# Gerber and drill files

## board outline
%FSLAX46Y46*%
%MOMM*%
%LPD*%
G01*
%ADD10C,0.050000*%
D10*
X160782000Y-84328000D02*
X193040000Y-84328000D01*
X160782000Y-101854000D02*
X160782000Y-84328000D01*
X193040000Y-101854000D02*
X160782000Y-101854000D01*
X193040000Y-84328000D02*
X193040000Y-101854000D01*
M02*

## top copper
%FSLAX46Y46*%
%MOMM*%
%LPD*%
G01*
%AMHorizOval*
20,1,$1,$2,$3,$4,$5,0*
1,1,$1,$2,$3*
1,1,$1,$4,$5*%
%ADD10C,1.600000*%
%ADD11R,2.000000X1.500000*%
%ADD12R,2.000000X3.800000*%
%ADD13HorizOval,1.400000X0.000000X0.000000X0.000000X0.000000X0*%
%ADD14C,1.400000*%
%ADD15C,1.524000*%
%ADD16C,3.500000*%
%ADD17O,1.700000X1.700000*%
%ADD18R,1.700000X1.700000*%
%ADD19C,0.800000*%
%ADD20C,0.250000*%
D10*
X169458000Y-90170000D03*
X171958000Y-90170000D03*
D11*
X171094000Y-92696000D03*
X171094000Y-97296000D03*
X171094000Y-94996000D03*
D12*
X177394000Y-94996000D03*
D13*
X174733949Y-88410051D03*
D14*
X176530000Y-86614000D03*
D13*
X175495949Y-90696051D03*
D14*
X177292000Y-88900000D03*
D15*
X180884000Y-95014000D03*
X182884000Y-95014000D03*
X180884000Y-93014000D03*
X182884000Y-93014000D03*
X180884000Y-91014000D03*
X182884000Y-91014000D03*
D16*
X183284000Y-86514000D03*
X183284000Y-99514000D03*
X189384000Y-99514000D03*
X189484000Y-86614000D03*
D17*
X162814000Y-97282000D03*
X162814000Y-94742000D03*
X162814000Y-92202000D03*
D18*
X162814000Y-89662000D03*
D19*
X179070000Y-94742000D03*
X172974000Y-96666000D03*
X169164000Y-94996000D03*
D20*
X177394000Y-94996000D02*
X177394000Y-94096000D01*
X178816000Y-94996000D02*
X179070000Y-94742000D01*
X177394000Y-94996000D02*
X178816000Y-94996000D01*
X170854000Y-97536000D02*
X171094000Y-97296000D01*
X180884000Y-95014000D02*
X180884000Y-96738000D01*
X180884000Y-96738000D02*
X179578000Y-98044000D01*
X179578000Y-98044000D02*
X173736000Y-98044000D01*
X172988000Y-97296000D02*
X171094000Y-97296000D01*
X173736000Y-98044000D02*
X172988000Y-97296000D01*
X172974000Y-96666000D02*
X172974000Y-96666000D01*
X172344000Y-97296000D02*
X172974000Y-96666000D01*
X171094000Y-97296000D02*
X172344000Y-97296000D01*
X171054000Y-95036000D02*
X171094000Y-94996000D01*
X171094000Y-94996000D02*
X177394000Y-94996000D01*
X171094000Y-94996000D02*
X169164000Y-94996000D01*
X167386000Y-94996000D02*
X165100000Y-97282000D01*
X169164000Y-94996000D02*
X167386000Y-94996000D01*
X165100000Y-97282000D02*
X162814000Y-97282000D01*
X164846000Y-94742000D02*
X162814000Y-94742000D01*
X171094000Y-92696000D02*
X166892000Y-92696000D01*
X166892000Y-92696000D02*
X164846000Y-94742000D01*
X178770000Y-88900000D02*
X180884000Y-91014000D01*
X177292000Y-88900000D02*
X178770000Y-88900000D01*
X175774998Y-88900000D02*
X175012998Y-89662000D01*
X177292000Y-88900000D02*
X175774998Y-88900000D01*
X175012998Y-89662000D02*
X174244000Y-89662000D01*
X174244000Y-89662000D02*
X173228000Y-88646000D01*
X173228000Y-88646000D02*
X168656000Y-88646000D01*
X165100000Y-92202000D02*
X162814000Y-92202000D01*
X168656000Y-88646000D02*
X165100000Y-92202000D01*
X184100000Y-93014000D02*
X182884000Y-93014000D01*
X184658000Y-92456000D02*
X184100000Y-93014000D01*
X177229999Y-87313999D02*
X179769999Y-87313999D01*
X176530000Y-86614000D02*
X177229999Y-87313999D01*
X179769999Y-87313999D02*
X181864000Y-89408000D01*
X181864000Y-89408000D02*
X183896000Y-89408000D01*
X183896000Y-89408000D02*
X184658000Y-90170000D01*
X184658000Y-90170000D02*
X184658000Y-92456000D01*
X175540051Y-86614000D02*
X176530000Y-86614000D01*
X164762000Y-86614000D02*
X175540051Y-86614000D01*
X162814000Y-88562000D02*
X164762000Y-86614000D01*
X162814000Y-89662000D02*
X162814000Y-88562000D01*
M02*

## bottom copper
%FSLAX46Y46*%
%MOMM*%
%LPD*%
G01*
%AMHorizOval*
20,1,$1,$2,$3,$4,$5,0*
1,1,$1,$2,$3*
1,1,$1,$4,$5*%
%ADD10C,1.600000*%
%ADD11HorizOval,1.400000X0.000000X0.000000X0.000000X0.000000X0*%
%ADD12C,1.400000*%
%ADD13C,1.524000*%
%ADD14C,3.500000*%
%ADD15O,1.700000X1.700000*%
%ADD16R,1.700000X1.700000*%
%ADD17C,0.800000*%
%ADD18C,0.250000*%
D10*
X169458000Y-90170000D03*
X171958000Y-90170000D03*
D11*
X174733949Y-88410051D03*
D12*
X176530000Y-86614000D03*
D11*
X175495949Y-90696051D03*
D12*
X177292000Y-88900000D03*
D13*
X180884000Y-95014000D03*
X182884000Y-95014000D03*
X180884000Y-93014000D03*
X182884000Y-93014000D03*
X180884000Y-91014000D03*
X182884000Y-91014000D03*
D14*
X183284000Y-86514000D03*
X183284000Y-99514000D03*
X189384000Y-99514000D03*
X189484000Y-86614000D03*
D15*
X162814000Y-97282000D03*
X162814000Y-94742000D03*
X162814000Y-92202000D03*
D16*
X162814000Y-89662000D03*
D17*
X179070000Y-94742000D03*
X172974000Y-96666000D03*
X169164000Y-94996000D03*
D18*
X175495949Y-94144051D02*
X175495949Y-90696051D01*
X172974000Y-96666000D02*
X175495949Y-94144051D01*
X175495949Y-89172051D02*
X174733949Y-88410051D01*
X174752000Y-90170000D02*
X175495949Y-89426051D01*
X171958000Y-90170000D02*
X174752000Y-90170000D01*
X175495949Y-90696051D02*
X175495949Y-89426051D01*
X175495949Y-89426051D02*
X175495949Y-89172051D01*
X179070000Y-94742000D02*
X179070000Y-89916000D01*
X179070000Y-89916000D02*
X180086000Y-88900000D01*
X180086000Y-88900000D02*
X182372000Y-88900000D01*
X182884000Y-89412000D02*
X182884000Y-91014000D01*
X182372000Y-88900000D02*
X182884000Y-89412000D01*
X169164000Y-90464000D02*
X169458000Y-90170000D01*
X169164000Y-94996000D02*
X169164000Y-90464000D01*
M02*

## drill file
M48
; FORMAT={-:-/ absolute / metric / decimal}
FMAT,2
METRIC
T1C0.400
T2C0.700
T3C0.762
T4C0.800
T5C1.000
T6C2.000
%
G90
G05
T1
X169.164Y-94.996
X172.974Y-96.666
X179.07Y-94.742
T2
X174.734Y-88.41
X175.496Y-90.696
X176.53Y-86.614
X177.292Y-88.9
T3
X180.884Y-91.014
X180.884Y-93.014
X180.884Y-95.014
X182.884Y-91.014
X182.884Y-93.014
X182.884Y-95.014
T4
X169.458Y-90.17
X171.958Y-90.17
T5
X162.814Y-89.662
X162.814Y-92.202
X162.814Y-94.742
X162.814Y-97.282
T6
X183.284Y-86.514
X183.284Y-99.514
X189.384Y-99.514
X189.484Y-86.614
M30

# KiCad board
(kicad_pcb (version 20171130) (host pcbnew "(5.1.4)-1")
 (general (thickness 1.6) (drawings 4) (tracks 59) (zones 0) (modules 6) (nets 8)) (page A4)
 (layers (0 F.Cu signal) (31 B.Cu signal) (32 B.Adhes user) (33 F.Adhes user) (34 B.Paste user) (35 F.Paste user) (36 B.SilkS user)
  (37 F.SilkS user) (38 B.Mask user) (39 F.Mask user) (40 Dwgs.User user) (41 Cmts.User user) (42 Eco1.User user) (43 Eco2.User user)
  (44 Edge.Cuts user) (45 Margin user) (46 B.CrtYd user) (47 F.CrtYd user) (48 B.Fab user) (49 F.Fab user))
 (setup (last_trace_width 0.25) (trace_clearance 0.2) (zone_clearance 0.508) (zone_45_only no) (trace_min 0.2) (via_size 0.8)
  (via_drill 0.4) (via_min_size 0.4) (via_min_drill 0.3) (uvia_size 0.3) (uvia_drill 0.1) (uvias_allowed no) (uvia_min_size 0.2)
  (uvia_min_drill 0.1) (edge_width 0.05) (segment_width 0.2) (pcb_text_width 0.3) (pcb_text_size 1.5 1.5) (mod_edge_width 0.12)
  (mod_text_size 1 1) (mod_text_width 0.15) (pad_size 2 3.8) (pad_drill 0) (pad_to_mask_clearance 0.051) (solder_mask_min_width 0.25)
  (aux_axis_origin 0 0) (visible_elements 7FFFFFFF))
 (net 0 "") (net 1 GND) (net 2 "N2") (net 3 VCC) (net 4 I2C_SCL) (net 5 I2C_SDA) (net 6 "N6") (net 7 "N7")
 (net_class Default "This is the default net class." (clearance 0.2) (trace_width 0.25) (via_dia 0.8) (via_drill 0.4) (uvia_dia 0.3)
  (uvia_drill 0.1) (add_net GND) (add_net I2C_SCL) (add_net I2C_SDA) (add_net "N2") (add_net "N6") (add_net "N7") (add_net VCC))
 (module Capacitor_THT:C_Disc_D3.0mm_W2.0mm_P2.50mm (layer F.Cu) (at 171.958 90.17 180)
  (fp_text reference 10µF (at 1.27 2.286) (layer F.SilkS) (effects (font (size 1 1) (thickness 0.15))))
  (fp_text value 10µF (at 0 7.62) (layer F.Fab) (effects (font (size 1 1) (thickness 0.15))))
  (pad 2 thru_hole circle (at 2.5 0 180) (size 1.6 1.6) (drill 0.8) (layers *.Cu *.Mask) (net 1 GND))
  (pad 1 thru_hole circle (at 0 0 180) (size 1.6 1.6) (drill 0.8) (layers *.Cu *.Mask) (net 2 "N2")))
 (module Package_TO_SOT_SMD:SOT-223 (layer F.Cu) (at 174.244 94.996)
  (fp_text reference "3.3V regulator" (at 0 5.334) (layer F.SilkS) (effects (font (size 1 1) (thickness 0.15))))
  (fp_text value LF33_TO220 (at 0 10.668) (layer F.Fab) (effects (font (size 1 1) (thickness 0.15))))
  (pad 1 smd rect (at -3.15 -2.3) (size 2 1.5) (layers F.Cu F.Paste F.Mask) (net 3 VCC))
  (pad 3 smd rect (at -3.15 2.3) (size 2 1.5) (layers F.Cu F.Paste F.Mask) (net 2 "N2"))
  (pad 2 smd rect (at -3.15 0) (size 2 1.5) (layers F.Cu F.Paste F.Mask) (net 1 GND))
  (pad 4 smd rect (at 3.15 0) (size 2 3.8) (layers F.Cu F.Paste F.Mask) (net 1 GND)))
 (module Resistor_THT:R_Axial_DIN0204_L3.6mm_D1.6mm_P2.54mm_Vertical (layer F.Cu) (at 176.53 86.614 225)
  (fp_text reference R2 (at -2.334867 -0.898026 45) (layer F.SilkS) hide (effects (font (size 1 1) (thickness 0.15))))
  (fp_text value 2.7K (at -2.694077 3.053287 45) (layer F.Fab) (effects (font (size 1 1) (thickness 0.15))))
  (pad 2 thru_hole oval (at 2.54 0 225) (size 1.4 1.4) (drill 0.7) (layers *.Cu *.Mask) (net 2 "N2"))
  (pad 1 thru_hole circle (at 0 0 225) (size 1.4 1.4) (drill 0.7) (layers *.Cu *.Mask) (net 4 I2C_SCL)))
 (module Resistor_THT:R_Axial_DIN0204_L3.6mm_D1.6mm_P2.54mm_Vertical (layer F.Cu) (at 177.292 88.9 225)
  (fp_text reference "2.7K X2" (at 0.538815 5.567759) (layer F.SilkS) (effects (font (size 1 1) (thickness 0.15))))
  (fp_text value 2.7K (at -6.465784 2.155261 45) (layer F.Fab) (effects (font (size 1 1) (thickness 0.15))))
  (pad 2 thru_hole oval (at 2.54 0 225) (size 1.4 1.4) (drill 0.7) (layers *.Cu *.Mask) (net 2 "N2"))
  (pad 1 thru_hole circle (at 0 0 225) (size 1.4 1.4) (drill 0.7) (layers *.Cu *.Mask) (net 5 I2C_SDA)))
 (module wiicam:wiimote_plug (layer F.Cu) (at 180.884 93.014)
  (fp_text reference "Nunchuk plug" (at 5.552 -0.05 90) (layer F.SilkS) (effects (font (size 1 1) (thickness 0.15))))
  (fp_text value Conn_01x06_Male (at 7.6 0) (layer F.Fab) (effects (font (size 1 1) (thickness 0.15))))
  (pad 1 thru_hole circle (at 0 2) (size 1.524 1.524) (drill 0.762) (layers *.Cu *.Mask) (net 2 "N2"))
  (pad 2 thru_hole circle (at 2 2) (size 1.524 1.524) (drill 0.762) (layers *.Cu *.Mask) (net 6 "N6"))
  (pad 3 thru_hole circle (at 0 0) (size 1.524 1.524) (drill 0.762) (layers *.Cu *.Mask) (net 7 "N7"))
  (pad 4 thru_hole circle (at 2 0) (size 1.524 1.524) (drill 0.762) (layers *.Cu *.Mask) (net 4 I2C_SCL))
  (pad 5 thru_hole circle (at 0 -2) (size 1.524 1.524) (drill 0.762) (layers *.Cu *.Mask) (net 5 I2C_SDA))
  (pad 6 thru_hole circle (at 2 -2) (size 1.524 1.524) (drill 0.762) (layers *.Cu *.Mask) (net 1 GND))
  (pad NC thru_hole circle (at 2.4 -6.5) (size 3.5 3.5) (drill 2) (layers *.Cu *.Mask))
  (pad NC thru_hole circle (at 2.4 6.5) (size 3.5 3.5) (drill 2) (layers *.Cu *.Mask))
  (pad NC thru_hole circle (at 8.5 6.5) (size 3.5 3.5) (drill 2) (layers *.Cu *.Mask))
  (pad NC thru_hole circle (at 8.6 -6.4) (size 3.5 3.5) (drill 2) (layers *.Cu *.Mask)))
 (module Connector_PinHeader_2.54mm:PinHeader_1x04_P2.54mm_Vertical (layer F.Cu) (at 162.814 89.662)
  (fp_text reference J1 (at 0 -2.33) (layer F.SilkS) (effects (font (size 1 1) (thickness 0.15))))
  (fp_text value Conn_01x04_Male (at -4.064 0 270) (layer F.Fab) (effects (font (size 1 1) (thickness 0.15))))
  (pad 4 thru_hole oval (at 0 7.62) (size 1.7 1.7) (drill 1) (layers *.Cu *.Mask) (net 1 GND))
  (pad 3 thru_hole oval (at 0 5.08) (size 1.7 1.7) (drill 1) (layers *.Cu *.Mask) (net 3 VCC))
  (pad 2 thru_hole oval (at 0 2.54) (size 1.7 1.7) (drill 1) (layers *.Cu *.Mask) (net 5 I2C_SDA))
  (pad 1 thru_hole rect (at 0 0) (size 1.7 1.7) (drill 1) (layers *.Cu *.Mask) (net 4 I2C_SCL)))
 (gr_line (start 160.782 84.328) (end 193.04 84.328) (layer Edge.Cuts) (width 0.05))
 (gr_line (start 160.782 101.854) (end 160.782 84.328) (layer Edge.Cuts) (width 0.05))
 (gr_line (start 193.04 101.854) (end 160.782 101.854) (layer Edge.Cuts) (width 0.05))
 (gr_line (start 193.04 84.328) (end 193.04 101.854) (layer Edge.Cuts) (width 0.05))
 (segment (start 177.394 94.996) (end 177.394 94.096) (width 0.25) (layer F.Cu) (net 1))
 (via (at 179.07 94.742) (size 0.8) (drill 0.4) (layers F.Cu B.Cu) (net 1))
 (segment (start 178.816 94.996) (end 179.07 94.742) (width 0.25) (layer F.Cu) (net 1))
 (segment (start 177.394 94.996) (end 178.816 94.996) (width 0.25) (layer F.Cu) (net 1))
 (segment (start 170.854 97.536) (end 171.094 97.296) (width 0.25) (layer F.Cu) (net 2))
 (segment (start 180.884 95.014) (end 180.884 96.738) (width 0.25) (layer F.Cu) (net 2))
 (segment (start 180.884 96.738) (end 179.578 98.044) (width 0.25) (layer F.Cu) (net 2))
 (segment (start 179.578 98.044) (end 173.736 98.044) (width 0.25) (layer F.Cu) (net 2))
 (segment (start 172.988 97.296) (end 171.094 97.296) (width 0.25) (layer F.Cu) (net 2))
 (segment (start 173.736 98.044) (end 172.988 97.296) (width 0.25) (layer F.Cu) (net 2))
 (segment (start 172.974 96.666) (end 172.974 96.666) (width 0.25) (layer F.Cu) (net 2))
 (via (at 172.974 96.666) (size 0.8) (drill 0.4) (layers F.Cu B.Cu) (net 2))
 (segment (start 172.344 97.296) (end 172.974 96.666) (width 0.25) (layer F.Cu) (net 2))
 (segment (start 171.094 97.296) (end 172.344 97.296) (width 0.25) (layer F.Cu) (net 2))
 (segment (start 175.495949 94.144051) (end 175.495949 90.696051) (width 0.25) (layer B.Cu) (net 2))
 (segment (start 172.974 96.666) (end 175.495949 94.144051) (width 0.25) (layer B.Cu) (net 2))
 (segment (start 175.495949 89.172051) (end 174.733949 88.410051) (width 0.25) (layer B.Cu) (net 2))
 (segment (start 174.752 90.17) (end 175.495949 89.426051) (width 0.25) (layer B.Cu) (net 2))
 (segment (start 171.958 90.17) (end 174.752 90.17) (width 0.25) (layer B.Cu) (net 2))
 (segment (start 175.495949 90.696051) (end 175.495949 89.426051) (width 0.25) (layer B.Cu) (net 2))
 (segment (start 175.495949 89.426051) (end 175.495949 89.172051) (width 0.25) (layer B.Cu) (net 2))
 (segment (start 171.054 95.036) (end 171.094 94.996) (width 0.25) (layer F.Cu) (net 1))
 (segment (start 179.07 94.742) (end 179.07 89.916) (width 0.25) (layer B.Cu) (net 1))
 (segment (start 179.07 89.916) (end 180.086 88.9) (width 0.25) (layer B.Cu) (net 1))
 (segment (start 180.086 88.9) (end 182.372 88.9) (width 0.25) (layer B.Cu) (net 1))
 (segment (start 182.884 89.412) (end 182.884 91.014) (width 0.25) (layer B.Cu) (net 1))
 (segment (start 182.372 88.9) (end 182.884 89.412) (width 0.25) (layer B.Cu) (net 1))
 (segment (start 171.094 94.996) (end 177.394 94.996) (width 0.25) (layer F.Cu) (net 1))
 (segment (start 171.094 94.996) (end 169.164 94.996) (width 0.25) (layer F.Cu) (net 1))
 (segment (start 167.386 94.996) (end 165.1 97.282) (width 0.25) (layer F.Cu) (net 1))
 (segment (start 169.164 94.996) (end 167.386 94.996) (width 0.25) (layer F.Cu) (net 1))
 (via (at 169.164 94.996) (size 0.8) (drill 0.4) (layers F.Cu B.Cu) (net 1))
 (segment (start 169.164 90.464) (end 169.458 90.17) (width 0.25) (layer B.Cu) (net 1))
 (segment (start 169.164 94.996) (end 169.164 90.464) (width 0.25) (layer B.Cu) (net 1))
 (segment (start 165.1 97.282) (end 162.814 97.282) (width 0.25) (layer F.Cu) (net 1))
 (segment (start 164.846 94.742) (end 162.814 94.742) (width 0.25) (layer F.Cu) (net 3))
 (segment (start 171.094 92.696) (end 166.892 92.696) (width 0.25) (layer F.Cu) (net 3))
 (segment (start 166.892 92.696) (end 164.846 94.742) (width 0.25) (layer F.Cu) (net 3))
 (segment (start 178.77 88.9) (end 180.884 91.014) (width 0.25) (layer F.Cu) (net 5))
 (segment (start 177.292 88.9) (end 178.77 88.9) (width 0.25) (layer F.Cu) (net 5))
 (segment (start 175.774998 88.9) (end 175.012998 89.662) (width 0.25) (layer F.Cu) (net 5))
 (segment (start 177.292 88.9) (end 175.774998 88.9) (width 0.25) (layer F.Cu) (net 5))
 (segment (start 175.012998 89.662) (end 174.244 89.662) (width 0.25) (layer F.Cu) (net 5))
 (segment (start 174.244 89.662) (end 173.228 88.646) (width 0.25) (layer F.Cu) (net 5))
 (segment (start 173.228 88.646) (end 168.656 88.646) (width 0.25) (layer F.Cu) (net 5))
 (segment (start 165.1 92.202) (end 162.814 92.202) (width 0.25) (layer F.Cu) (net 5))
 (segment (start 168.656 88.646) (end 165.1 92.202) (width 0.25) (layer F.Cu) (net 5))
 (segment (start 184.1 93.014) (end 182.884 93.014) (width 0.25) (layer F.Cu) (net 4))
 (segment (start 184.658 92.456) (end 184.1 93.014) (width 0.25) (layer F.Cu) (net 4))
 (segment (start 177.229999 87.313999) (end 179.769999 87.313999) (width 0.25) (layer F.Cu) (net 4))
 (segment (start 176.53 86.614) (end 177.229999 87.313999) (width 0.25) (layer F.Cu) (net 4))
 (segment (start 179.769999 87.313999) (end 181.864 89.408) (width 0.25) (layer F.Cu) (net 4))
 (segment (start 181.864 89.408) (end 183.896 89.408) (width 0.25) (layer F.Cu) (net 4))
 (segment (start 183.896 89.408) (end 184.658 90.17) (width 0.25) (layer F.Cu) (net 4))
 (segment (start 184.658 90.17) (end 184.658 92.456) (width 0.25) (layer F.Cu) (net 4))
 (segment (start 175.540051 86.614) (end 176.53 86.614) (width 0.25) (layer F.Cu) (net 4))
 (segment (start 164.762 86.614) (end 175.540051 86.614) (width 0.25) (layer F.Cu) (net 4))
 (segment (start 162.814 88.562) (end 164.762 86.614) (width 0.25) (layer F.Cu) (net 4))
 (segment (start 162.814 89.662) (end 162.814 88.562) (width 0.25) (layer F.Cu) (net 4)))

